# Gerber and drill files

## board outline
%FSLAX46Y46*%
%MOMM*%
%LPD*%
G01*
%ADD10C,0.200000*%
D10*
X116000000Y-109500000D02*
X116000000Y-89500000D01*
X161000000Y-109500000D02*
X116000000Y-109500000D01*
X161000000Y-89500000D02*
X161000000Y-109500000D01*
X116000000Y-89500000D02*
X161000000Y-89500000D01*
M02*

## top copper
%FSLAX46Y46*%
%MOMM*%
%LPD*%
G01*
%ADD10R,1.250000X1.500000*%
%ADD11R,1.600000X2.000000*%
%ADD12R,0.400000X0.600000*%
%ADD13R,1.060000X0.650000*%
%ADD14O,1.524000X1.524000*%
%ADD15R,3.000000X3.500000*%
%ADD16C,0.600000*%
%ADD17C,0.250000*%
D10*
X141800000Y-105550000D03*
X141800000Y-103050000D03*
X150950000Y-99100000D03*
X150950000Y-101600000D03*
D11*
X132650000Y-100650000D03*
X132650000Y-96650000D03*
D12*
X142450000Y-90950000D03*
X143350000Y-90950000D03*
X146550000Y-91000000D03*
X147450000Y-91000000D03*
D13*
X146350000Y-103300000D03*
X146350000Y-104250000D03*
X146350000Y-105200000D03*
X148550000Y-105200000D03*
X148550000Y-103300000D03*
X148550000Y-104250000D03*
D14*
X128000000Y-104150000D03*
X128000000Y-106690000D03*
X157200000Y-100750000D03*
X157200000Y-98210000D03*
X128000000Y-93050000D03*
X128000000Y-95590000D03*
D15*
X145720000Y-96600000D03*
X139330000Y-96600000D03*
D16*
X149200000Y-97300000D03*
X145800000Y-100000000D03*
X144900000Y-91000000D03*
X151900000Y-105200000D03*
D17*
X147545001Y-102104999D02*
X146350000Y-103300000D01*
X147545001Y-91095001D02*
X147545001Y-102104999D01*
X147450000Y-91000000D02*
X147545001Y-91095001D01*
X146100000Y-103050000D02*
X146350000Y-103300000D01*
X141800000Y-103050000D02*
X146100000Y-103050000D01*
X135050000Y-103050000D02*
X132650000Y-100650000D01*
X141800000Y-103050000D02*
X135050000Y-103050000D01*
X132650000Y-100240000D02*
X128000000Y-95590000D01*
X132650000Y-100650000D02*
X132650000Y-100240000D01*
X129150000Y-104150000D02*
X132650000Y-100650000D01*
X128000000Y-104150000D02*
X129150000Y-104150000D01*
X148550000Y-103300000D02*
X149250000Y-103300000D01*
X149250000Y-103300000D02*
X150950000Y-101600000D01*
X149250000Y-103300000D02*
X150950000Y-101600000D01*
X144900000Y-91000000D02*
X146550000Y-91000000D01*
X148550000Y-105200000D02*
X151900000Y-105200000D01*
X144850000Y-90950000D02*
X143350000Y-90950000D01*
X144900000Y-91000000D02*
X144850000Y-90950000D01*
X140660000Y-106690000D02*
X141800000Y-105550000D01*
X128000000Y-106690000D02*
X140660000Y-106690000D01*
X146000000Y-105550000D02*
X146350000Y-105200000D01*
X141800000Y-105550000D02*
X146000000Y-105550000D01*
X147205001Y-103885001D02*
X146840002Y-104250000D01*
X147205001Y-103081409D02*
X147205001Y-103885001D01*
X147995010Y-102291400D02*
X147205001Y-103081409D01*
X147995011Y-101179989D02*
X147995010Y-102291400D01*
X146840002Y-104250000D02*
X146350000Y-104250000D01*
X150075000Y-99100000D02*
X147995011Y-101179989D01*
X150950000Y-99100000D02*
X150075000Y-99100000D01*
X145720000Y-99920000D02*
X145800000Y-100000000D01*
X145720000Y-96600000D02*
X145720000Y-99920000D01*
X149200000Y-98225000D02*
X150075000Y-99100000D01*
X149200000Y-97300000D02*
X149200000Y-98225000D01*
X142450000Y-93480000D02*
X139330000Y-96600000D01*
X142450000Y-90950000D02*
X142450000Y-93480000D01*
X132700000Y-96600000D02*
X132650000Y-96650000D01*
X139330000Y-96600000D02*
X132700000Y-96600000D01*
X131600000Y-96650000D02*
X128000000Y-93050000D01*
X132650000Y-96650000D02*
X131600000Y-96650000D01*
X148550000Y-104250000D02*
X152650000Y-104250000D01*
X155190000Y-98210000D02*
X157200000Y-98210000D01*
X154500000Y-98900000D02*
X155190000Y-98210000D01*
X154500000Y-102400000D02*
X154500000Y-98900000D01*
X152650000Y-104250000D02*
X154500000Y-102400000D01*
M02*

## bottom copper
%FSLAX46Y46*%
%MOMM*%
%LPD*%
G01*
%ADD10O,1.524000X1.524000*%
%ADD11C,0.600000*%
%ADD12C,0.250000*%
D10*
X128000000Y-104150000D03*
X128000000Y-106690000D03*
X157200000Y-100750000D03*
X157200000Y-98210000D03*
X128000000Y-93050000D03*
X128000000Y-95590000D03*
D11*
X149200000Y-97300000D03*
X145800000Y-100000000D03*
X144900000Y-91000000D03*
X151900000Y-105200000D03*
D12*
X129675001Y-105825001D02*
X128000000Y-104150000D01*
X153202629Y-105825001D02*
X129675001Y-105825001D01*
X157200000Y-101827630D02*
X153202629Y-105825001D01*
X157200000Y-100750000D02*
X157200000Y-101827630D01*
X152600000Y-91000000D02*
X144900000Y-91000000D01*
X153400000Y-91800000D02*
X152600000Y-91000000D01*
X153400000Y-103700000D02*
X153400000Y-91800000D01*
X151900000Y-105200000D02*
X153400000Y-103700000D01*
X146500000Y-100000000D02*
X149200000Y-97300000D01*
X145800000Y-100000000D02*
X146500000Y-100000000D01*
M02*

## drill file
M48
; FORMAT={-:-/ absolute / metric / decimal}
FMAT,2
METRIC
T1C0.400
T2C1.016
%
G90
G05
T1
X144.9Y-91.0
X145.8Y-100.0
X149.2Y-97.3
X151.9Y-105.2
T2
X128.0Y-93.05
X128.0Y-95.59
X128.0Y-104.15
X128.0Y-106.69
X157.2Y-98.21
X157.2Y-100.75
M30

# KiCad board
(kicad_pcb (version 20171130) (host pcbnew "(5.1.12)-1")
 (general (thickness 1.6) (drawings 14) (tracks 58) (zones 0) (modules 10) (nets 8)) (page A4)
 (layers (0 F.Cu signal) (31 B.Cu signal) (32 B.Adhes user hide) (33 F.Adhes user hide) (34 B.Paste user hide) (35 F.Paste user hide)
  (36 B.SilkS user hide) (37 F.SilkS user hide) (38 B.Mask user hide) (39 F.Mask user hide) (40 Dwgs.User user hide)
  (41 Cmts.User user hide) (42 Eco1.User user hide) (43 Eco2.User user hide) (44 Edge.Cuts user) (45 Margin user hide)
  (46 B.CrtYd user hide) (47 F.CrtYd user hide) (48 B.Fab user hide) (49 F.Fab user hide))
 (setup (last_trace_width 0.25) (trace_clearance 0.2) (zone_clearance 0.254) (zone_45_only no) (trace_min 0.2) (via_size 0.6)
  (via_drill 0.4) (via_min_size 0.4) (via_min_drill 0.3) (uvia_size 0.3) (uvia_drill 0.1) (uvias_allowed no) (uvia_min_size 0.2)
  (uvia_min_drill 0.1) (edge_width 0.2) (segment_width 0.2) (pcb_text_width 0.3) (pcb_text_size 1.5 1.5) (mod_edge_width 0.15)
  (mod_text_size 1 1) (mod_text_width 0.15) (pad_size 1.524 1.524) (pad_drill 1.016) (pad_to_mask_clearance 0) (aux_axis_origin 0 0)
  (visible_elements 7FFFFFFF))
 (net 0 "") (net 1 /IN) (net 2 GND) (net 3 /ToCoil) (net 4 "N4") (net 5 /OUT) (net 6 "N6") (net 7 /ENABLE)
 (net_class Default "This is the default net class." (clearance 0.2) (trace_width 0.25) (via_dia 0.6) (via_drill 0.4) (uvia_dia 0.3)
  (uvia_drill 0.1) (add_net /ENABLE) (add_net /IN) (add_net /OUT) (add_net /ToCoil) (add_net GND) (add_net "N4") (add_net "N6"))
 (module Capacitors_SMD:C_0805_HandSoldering (layer F.Cu) (at 141.8 104.3 90)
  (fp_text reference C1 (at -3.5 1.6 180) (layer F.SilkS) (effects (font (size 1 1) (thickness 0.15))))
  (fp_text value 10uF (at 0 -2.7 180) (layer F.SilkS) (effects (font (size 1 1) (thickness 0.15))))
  (pad 1 smd rect (at -1.25 0 90) (size 1.5 1.25) (layers F.Cu F.Paste F.Mask) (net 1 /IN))
  (pad 2 smd rect (at 1.25 0 90) (size 1.5 1.25) (layers F.Cu F.Paste F.Mask) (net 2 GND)))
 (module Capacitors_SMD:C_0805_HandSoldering (layer F.Cu) (at 150.95 100.35 270)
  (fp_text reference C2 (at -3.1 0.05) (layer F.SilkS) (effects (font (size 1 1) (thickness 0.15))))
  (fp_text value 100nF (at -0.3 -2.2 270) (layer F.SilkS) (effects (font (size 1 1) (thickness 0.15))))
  (pad 1 smd rect (at -1.25 0 270) (size 1.5 1.25) (layers F.Cu F.Paste F.Mask) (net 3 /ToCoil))
  (pad 2 smd rect (at 1.25 0 270) (size 1.5 1.25) (layers F.Cu F.Paste F.Mask) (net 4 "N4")))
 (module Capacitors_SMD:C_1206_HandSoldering (layer F.Cu) (at 132.65 98.65 90)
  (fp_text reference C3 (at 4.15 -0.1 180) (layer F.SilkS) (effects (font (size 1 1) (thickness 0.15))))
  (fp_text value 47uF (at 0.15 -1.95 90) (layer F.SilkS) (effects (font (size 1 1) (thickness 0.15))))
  (pad 1 smd rect (at -2 0 90) (size 2 1.6) (layers F.Cu F.Paste F.Mask) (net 2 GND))
  (pad 2 smd rect (at 2 0 90) (size 2 1.6) (layers F.Cu F.Paste F.Mask) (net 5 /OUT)))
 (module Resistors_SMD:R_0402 (layer F.Cu) (at 142.9 90.95)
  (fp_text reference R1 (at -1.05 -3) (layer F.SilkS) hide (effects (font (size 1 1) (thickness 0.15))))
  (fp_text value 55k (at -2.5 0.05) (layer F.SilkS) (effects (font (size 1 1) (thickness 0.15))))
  (pad 1 smd rect (at -0.45 0) (size 0.4 0.6) (layers F.Cu F.Paste F.Mask) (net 5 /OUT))
  (pad 2 smd rect (at 0.45 0) (size 0.4 0.6) (layers F.Cu F.Paste F.Mask) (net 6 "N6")))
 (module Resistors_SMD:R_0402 (layer F.Cu) (at 147 91)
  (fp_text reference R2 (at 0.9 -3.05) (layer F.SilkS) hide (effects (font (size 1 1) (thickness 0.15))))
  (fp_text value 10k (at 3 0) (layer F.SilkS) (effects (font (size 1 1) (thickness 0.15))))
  (pad 1 smd rect (at -0.45 0) (size 0.4 0.6) (layers F.Cu F.Paste F.Mask) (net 6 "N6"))
  (pad 2 smd rect (at 0.45 0) (size 0.4 0.6) (layers F.Cu F.Paste F.Mask) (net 2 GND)))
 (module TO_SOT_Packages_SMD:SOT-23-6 (layer F.Cu) (at 147.45 104.25)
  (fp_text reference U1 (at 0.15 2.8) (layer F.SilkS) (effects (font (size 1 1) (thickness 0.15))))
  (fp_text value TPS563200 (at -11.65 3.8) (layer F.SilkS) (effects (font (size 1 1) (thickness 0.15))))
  (pad 1 smd rect (at -1.1 -0.95) (size 1.06 0.65) (layers F.Cu F.Paste F.Mask) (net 2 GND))
  (pad 2 smd rect (at -1.1 0) (size 1.06 0.65) (layers F.Cu F.Paste F.Mask) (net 3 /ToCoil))
  (pad 3 smd rect (at -1.1 0.95) (size 1.06 0.65) (layers F.Cu F.Paste F.Mask) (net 1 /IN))
  (pad 4 smd rect (at 1.1 0.95) (size 1.06 0.65) (layers F.Cu F.Paste F.Mask) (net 6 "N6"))
  (pad 6 smd rect (at 1.1 -0.95) (size 1.06 0.65) (layers F.Cu F.Paste F.Mask) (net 4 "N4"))
  (pad 5 smd rect (at 1.1 0) (size 1.06 0.65) (layers F.Cu F.Paste F.Mask) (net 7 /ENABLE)))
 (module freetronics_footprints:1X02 (layer F.Cu) (at 128 104.15 270)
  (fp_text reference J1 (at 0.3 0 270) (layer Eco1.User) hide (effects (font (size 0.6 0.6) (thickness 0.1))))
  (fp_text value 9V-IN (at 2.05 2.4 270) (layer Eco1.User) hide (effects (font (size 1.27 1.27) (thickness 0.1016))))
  (pad 1 thru_hole oval (at 0 0) (size 1.524 1.524) (drill 1.016) (layers *.Cu *.Mask) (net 2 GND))
  (pad 2 thru_hole oval (at 2.54 0) (size 1.524 1.524) (drill 1.016) (layers *.Cu *.Mask) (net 1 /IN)))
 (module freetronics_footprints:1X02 (layer F.Cu) (at 157.2 100.75 90)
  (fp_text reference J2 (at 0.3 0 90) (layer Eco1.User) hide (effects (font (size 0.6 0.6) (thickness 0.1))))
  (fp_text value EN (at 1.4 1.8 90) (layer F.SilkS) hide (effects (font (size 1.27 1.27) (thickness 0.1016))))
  (pad 1 thru_hole oval (at 0 0 180) (size 1.524 1.524) (drill 1.016) (layers *.Cu *.Mask) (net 2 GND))
  (pad 2 thru_hole oval (at 2.54 0 180) (size 1.524 1.524) (drill 1.016) (layers *.Cu *.Mask) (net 7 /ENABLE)))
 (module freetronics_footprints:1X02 (layer F.Cu) (at 128 93.05 270)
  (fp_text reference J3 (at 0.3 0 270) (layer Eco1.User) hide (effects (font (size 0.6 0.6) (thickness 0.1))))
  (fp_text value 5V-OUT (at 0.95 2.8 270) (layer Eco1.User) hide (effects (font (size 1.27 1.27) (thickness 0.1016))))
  (pad 1 thru_hole oval (at 0 0) (size 1.524 1.524) (drill 1.016) (layers *.Cu *.Mask) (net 5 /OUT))
  (pad 2 thru_hole oval (at 2.54 0) (size 1.524 1.524) (drill 1.016) (layers *.Cu *.Mask) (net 2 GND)))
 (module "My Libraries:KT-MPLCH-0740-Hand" (layer F.Cu) (at 142.4 96.6 180)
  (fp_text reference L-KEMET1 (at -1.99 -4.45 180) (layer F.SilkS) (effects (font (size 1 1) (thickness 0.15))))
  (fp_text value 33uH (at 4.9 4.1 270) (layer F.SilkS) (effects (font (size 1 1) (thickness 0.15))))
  (pad 1 smd rect (at -3.32 0 180) (size 3 3.5) (layers F.Cu F.Paste F.Mask) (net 3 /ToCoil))
  (pad 2 smd rect (at 3.07 0 180) (size 3 3.5) (layers F.Cu F.Paste F.Mask) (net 5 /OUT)))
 (gr_line (start 116 109.5) (end 116 89.5) (angle 90) (layer Edge.Cuts) (width 0.2))
 (gr_line (start 161 109.5) (end 116 109.5) (angle 90) (layer Edge.Cuts) (width 0.2))
 (gr_line (start 161 89.5) (end 161 109.5) (angle 90) (layer Edge.Cuts) (width 0.2))
 (gr_line (start 116 89.5) (end 161 89.5) (angle 90) (layer Edge.Cuts) (width 0.2))
 (via (at 149.2 97.3) (size 0.6) (drill 0.4) (layers F.Cu B.Cu) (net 3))
 (via (at 145.8 100) (size 0.6) (drill 0.4) (layers F.Cu B.Cu) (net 3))
 (segment (start 147.545001 102.104999) (end 146.35 103.3) (width 0.25) (layer F.Cu) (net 2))
 (segment (start 147.545001 91.095001) (end 147.545001 102.104999) (width 0.25) (layer F.Cu) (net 2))
 (segment (start 147.45 91) (end 147.545001 91.095001) (width 0.25) (layer F.Cu) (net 2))
 (segment (start 146.1 103.05) (end 146.35 103.3) (width 0.25) (layer F.Cu) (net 2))
 (segment (start 141.8 103.05) (end 146.1 103.05) (width 0.25) (layer F.Cu) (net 2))
 (segment (start 135.05 103.05) (end 132.65 100.65) (width 0.25) (layer F.Cu) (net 2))
 (segment (start 141.8 103.05) (end 135.05 103.05) (width 0.25) (layer F.Cu) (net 2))
 (segment (start 132.65 100.24) (end 128 95.59) (width 0.25) (layer F.Cu) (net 2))
 (segment (start 132.65 100.65) (end 132.65 100.24) (width 0.25) (layer F.Cu) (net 2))
 (segment (start 129.15 104.15) (end 132.65 100.65) (width 0.25) (layer F.Cu) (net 2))
 (segment (start 128 104.15) (end 129.15 104.15) (width 0.25) (layer F.Cu) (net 2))
 (segment (start 129.675001 105.825001) (end 128 104.15) (width 0.25) (layer B.Cu) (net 2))
 (segment (start 153.202629 105.825001) (end 129.675001 105.825001) (width 0.25) (layer B.Cu) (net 2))
 (segment (start 157.2 101.82763) (end 153.202629 105.825001) (width 0.25) (layer B.Cu) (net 2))
 (segment (start 157.2 100.75) (end 157.2 101.82763) (width 0.25) (layer B.Cu) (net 2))
 (segment (start 148.55 103.3) (end 149.25 103.3) (width 0.25) (layer F.Cu) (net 4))
 (segment (start 149.25 103.3) (end 150.95 101.6) (width 0.25) (layer F.Cu) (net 4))
 (segment (start 149.25 103.3) (end 150.95 101.6) (width 0.25) (layer F.Cu) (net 4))
 (segment (start 144.9 91) (end 146.55 91) (width 0.25) (layer F.Cu) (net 6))
 (segment (start 148.55 105.2) (end 151.9 105.2) (width 0.25) (layer F.Cu) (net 6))
 (segment (start 144.85 90.95) (end 143.35 90.95) (width 0.25) (layer F.Cu) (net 6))
 (segment (start 144.9 91) (end 144.85 90.95) (width 0.25) (layer F.Cu) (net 6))
 (segment (start 152.6 91) (end 144.9 91) (width 0.25) (layer B.Cu) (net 6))
 (segment (start 153.4 91.8) (end 152.6 91) (width 0.25) (layer B.Cu) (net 6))
 (segment (start 153.4 103.7) (end 153.4 91.8) (width 0.25) (layer B.Cu) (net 6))
 (segment (start 151.9 105.2) (end 153.4 103.7) (width 0.25) (layer B.Cu) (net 6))
 (via (at 144.9 91) (size 0.6) (drill 0.4) (layers F.Cu B.Cu) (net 6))
 (via (at 151.9 105.2) (size 0.6) (drill 0.4) (layers F.Cu B.Cu) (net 6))
 (segment (start 140.66 106.69) (end 141.8 105.55) (width 0.25) (layer F.Cu) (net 1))
 (segment (start 128 106.69) (end 140.66 106.69) (width 0.25) (layer F.Cu) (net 1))
 (segment (start 146 105.55) (end 146.35 105.2) (width 0.25) (layer F.Cu) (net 1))
 (segment (start 141.8 105.55) (end 146 105.55) (width 0.25) (layer F.Cu) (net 1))
 (segment (start 147.205001 103.885001) (end 146.840002 104.25) (width 0.25) (layer F.Cu) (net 3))
 (segment (start 147.205001 103.081409) (end 147.205001 103.885001) (width 0.25) (layer F.Cu) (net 3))
 (segment (start 147.99501 102.2914) (end 147.205001 103.081409) (width 0.25) (layer F.Cu) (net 3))
 (segment (start 147.995011 101.179989) (end 147.99501 102.2914) (width 0.25) (layer F.Cu) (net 3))
 (segment (start 146.840002 104.25) (end 146.35 104.25) (width 0.25) (layer F.Cu) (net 3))
 (segment (start 150.075 99.1) (end 147.995011 101.179989) (width 0.25) (layer F.Cu) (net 3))
 (segment (start 150.95 99.1) (end 150.075 99.1) (width 0.25) (layer F.Cu) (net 3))
 (segment (start 145.72 99.92) (end 145.8 100) (width 0.25) (layer F.Cu) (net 3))
 (segment (start 145.72 96.6) (end 145.72 99.92) (width 0.25) (layer F.Cu) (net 3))
 (segment (start 149.2 98.225) (end 150.075 99.1) (width 0.25) (layer F.Cu) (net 3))
 (segment (start 149.2 97.3) (end 149.2 98.225) (width 0.25) (layer F.Cu) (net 3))
 (segment (start 146.5 100) (end 149.2 97.3) (width 0.25) (layer B.Cu) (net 3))
 (segment (start 145.8 100) (end 146.5 100) (width 0.25) (layer B.Cu) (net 3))
 (segment (start 142.45 93.48) (end 139.33 96.6) (width 0.25) (layer F.Cu) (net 5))
 (segment (start 142.45 90.95) (end 142.45 93.48) (width 0.25) (layer F.Cu) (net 5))
 (segment (start 132.7 96.6) (end 132.65 96.65) (width 0.25) (layer F.Cu) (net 5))
 (segment (start 139.33 96.6) (end 132.7 96.6) (width 0.25) (layer F.Cu) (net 5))
 (segment (start 131.6 96.65) (end 128 93.05) (width 0.25) (layer F.Cu) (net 5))
 (segment (start 132.65 96.65) (end 131.6 96.65) (width 0.25) (layer F.Cu) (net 5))
 (segment (start 148.55 104.25) (end 152.65 104.25) (width 0.25) (layer F.Cu) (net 7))
 (segment (start 155.19 98.21) (end 157.2 98.21) (width 0.25) (layer F.Cu) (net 7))
 (segment (start 154.5 98.9) (end 155.19 98.21) (width 0.25) (layer F.Cu) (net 7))
 (segment (start 154.5 102.4) (end 154.5 98.9) (width 0.25) (layer F.Cu) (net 7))
 (segment (start 152.65 104.25) (end 154.5 102.4) (width 0.25) (layer F.Cu) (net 7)))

